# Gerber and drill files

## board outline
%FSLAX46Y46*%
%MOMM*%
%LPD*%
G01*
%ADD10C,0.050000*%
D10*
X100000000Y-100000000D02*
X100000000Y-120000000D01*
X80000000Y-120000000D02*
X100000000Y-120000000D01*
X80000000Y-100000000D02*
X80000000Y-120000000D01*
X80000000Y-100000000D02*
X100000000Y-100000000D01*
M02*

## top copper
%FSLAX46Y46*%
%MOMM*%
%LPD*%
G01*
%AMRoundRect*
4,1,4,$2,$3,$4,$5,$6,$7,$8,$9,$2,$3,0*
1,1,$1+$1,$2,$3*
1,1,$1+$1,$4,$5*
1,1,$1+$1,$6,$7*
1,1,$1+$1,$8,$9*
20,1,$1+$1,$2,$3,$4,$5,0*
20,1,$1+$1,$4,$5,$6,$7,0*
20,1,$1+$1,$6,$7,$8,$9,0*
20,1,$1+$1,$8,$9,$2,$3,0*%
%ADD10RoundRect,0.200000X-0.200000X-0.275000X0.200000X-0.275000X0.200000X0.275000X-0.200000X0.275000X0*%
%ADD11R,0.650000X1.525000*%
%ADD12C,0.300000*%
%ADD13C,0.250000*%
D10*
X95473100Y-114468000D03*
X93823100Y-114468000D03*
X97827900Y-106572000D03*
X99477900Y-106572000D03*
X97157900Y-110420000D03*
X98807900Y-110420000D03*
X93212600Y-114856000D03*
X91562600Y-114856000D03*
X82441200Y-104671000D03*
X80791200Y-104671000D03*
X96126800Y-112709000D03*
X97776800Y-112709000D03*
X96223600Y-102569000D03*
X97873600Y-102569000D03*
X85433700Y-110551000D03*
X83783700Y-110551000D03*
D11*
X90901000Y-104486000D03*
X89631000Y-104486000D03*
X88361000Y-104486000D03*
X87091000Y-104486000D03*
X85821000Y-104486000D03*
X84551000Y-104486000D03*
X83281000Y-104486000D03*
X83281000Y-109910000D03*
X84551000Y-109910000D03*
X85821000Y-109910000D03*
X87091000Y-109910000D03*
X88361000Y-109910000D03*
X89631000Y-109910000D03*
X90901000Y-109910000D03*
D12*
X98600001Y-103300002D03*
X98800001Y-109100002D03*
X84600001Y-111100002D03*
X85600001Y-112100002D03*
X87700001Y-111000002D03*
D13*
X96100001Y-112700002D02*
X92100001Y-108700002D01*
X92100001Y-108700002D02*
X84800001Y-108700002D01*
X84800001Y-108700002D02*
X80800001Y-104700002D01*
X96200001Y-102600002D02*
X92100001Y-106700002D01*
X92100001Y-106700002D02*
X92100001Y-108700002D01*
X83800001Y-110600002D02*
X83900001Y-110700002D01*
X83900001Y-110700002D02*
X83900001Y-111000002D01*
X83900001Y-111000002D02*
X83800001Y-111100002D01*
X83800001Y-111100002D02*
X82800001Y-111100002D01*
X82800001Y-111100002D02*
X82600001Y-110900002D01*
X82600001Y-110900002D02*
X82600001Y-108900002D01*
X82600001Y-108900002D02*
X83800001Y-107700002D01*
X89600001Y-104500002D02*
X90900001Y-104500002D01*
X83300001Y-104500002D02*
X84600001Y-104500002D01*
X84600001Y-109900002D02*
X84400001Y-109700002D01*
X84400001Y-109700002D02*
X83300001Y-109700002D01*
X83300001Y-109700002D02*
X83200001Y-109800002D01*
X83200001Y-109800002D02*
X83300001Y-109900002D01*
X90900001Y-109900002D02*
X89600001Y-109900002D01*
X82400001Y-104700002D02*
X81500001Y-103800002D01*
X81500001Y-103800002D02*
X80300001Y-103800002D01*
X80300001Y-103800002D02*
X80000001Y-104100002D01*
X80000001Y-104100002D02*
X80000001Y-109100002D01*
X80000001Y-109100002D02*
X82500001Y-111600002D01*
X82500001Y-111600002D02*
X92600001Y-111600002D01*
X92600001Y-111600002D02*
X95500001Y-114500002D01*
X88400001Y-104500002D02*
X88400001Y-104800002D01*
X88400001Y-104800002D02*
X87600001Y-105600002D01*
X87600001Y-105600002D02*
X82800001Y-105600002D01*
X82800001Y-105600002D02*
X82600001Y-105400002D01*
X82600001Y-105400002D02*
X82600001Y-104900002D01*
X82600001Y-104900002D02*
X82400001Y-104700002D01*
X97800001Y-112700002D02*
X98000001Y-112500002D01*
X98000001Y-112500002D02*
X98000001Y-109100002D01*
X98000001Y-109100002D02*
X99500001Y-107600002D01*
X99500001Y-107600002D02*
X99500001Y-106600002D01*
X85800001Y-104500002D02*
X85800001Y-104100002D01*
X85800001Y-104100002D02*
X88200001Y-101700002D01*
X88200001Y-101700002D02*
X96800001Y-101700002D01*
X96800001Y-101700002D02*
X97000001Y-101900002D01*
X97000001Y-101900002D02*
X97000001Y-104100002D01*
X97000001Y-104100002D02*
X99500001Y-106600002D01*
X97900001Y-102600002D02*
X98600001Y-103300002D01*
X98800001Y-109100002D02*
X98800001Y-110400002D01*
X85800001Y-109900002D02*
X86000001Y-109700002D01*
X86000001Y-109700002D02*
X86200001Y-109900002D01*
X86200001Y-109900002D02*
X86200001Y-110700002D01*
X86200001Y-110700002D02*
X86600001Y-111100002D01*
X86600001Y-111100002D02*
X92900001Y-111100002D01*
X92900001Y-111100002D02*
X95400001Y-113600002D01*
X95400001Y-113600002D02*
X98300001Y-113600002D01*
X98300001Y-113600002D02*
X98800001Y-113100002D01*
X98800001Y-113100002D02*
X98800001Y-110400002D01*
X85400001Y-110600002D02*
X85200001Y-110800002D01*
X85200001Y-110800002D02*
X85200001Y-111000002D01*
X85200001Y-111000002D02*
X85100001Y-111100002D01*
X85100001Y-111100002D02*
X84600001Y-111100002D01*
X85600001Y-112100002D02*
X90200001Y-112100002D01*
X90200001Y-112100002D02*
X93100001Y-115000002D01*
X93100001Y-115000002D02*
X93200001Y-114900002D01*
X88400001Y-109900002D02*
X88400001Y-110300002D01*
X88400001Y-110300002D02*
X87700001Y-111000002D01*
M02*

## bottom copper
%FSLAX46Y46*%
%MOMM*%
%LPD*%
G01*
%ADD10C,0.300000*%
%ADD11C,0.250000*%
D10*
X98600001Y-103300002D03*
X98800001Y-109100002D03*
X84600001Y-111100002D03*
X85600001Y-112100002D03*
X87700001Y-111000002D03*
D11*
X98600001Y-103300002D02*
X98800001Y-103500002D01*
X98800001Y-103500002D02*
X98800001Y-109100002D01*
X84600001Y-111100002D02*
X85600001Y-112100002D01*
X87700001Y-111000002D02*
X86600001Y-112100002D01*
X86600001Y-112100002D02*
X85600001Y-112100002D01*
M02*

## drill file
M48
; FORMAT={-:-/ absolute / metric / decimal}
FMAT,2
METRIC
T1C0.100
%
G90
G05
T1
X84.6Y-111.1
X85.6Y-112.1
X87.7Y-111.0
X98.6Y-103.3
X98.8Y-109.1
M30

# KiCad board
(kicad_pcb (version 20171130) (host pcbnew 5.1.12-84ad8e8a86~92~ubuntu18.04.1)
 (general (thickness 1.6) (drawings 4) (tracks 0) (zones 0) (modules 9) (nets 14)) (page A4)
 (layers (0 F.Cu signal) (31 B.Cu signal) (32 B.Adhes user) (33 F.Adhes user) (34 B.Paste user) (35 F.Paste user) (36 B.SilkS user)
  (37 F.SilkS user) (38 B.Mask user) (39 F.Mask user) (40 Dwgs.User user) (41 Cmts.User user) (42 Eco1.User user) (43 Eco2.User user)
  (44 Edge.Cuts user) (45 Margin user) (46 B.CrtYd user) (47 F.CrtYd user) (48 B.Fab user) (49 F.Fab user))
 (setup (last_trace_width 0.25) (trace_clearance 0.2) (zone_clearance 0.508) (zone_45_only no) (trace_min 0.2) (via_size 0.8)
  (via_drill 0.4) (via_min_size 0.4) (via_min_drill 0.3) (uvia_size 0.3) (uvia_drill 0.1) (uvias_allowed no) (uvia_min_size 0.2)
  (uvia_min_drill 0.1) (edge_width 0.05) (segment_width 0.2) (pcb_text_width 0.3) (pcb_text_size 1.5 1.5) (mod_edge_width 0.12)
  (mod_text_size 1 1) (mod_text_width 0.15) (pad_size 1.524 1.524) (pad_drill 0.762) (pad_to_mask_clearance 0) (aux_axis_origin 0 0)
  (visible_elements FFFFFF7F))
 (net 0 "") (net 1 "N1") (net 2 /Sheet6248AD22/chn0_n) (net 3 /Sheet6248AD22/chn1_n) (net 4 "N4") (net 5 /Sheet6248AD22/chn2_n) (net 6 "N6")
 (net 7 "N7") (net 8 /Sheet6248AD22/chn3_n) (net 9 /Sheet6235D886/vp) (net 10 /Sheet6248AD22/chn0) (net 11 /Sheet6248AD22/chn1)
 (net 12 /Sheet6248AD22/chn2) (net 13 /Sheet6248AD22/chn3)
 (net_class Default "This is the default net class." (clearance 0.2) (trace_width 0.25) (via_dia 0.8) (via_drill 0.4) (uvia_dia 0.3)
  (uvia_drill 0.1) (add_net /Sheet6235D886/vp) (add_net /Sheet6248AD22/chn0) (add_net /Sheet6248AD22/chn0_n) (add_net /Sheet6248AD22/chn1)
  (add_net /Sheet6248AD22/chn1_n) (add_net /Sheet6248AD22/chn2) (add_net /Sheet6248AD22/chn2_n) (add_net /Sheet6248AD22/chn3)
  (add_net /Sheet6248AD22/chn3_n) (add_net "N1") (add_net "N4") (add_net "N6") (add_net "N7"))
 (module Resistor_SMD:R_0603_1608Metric (layer F.Cu) (at 94.648100 114.468000)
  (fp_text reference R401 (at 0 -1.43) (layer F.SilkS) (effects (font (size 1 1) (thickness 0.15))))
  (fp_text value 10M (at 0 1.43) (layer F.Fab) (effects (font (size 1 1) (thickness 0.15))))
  (pad 2 smd roundrect (at 0.825 0) (size 0.8 0.95) (layers F.Cu F.Mask F.Paste) (roundrect_rratio 0.25) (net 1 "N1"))
  (pad 1 smd roundrect (at -0.825 0) (size 0.8 0.95) (layers F.Cu F.Mask F.Paste) (roundrect_rratio 0.25) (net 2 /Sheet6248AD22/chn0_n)))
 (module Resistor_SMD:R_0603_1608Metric (layer F.Cu) (at 98.652900 106.572000)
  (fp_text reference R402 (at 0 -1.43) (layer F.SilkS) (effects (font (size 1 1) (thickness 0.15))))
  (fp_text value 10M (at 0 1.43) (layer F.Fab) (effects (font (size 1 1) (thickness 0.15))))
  (pad 1 smd roundrect (at -0.825 0) (size 0.8 0.95) (layers F.Cu F.Mask F.Paste) (roundrect_rratio 0.25) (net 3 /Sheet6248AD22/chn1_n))
  (pad 2 smd roundrect (at 0.825 0) (size 0.8 0.95) (layers F.Cu F.Mask F.Paste) (roundrect_rratio 0.25) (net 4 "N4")))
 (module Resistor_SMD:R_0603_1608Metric (layer F.Cu) (at 97.982900 110.420000)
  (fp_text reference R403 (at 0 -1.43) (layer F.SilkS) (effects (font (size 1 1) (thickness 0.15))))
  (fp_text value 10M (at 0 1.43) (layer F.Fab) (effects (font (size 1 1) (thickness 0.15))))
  (pad 1 smd roundrect (at -0.825 0) (size 0.8 0.95) (layers F.Cu F.Mask F.Paste) (roundrect_rratio 0.25) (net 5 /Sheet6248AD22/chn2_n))
  (pad 2 smd roundrect (at 0.825 0) (size 0.8 0.95) (layers F.Cu F.Mask F.Paste) (roundrect_rratio 0.25) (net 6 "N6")))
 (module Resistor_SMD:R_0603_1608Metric (layer F.Cu) (at 92.387600 114.856000)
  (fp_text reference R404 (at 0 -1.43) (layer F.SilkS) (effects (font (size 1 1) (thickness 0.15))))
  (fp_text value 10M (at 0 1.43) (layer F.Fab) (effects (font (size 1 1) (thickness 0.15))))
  (pad 2 smd roundrect (at 0.825 0) (size 0.8 0.95) (layers F.Cu F.Mask F.Paste) (roundrect_rratio 0.25) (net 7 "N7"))
  (pad 1 smd roundrect (at -0.825 0) (size 0.8 0.95) (layers F.Cu F.Mask F.Paste) (roundrect_rratio 0.25) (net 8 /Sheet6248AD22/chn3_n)))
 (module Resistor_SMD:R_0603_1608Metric (layer F.Cu) (at 81.616200 104.671000)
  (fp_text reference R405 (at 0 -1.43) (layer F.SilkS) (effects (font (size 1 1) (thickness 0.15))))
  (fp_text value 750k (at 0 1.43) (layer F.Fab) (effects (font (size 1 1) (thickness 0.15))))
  (pad 2 smd roundrect (at 0.825 0) (size 0.8 0.95) (layers F.Cu F.Mask F.Paste) (roundrect_rratio 0.25) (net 1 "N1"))
  (pad 1 smd roundrect (at -0.825 0) (size 0.8 0.95) (layers F.Cu F.Mask F.Paste) (roundrect_rratio 0.25) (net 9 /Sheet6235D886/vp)))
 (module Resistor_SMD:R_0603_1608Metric (layer F.Cu) (at 96.951800 112.709000)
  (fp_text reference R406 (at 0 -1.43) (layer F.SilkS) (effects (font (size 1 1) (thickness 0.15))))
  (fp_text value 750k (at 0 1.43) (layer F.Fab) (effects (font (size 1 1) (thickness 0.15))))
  (pad 1 smd roundrect (at -0.825 0) (size 0.8 0.95) (layers F.Cu F.Mask F.Paste) (roundrect_rratio 0.25) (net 9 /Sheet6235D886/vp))
  (pad 2 smd roundrect (at 0.825 0) (size 0.8 0.95) (layers F.Cu F.Mask F.Paste) (roundrect_rratio 0.25) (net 4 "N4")))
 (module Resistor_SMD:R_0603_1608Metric (layer F.Cu) (at 97.048600 102.569000)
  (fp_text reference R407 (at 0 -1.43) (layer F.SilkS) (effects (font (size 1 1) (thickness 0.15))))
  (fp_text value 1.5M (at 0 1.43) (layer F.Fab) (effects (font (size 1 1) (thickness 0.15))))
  (pad 1 smd roundrect (at -0.825 0) (size 0.8 0.95) (layers F.Cu F.Mask F.Paste) (roundrect_rratio 0.25) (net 9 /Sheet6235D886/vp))
  (pad 2 smd roundrect (at 0.825 0) (size 0.8 0.95) (layers F.Cu F.Mask F.Paste) (roundrect_rratio 0.25) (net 6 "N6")))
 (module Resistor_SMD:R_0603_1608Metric (layer F.Cu) (at 84.608700 110.551000)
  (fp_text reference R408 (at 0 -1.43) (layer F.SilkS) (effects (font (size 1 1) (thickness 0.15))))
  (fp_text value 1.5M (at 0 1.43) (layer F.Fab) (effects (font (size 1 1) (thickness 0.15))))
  (pad 2 smd roundrect (at 0.825 0) (size 0.8 0.95) (layers F.Cu F.Mask F.Paste) (roundrect_rratio 0.25) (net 7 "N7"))
  (pad 1 smd roundrect (at -0.825 0) (size 0.8 0.95) (layers F.Cu F.Mask F.Paste) (roundrect_rratio 0.25) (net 9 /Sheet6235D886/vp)))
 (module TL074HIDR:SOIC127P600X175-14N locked (layer F.Cu) (at 87.091000 107.198000 270.000000)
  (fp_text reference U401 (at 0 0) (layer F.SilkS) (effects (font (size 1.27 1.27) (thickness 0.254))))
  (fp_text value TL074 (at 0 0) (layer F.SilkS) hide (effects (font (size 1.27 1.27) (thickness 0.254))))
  (pad 1 smd rect (at -2.712 -3.81) (size 0.65 1.525) (layers F.Cu F.Mask F.Paste) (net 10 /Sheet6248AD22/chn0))
  (pad 2 smd rect (at -2.712 -2.54) (size 0.65 1.525) (layers F.Cu F.Mask F.Paste) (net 10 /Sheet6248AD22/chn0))
  (pad 3 smd rect (at -2.712 -1.27) (size 0.65 1.525) (layers F.Cu F.Mask F.Paste) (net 1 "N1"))
  (pad 4 smd rect (at -2.712 0) (size 0.65 1.525) (layers F.Cu F.Mask F.Paste))
  (pad 5 smd rect (at -2.712 1.27) (size 0.65 1.525) (layers F.Cu F.Mask F.Paste) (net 4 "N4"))
  (pad 6 smd rect (at -2.712 2.54) (size 0.65 1.525) (layers F.Cu F.Mask F.Paste) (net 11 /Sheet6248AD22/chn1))
  (pad 7 smd rect (at -2.712 3.81) (size 0.65 1.525) (layers F.Cu F.Mask F.Paste) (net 11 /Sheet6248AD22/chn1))
  (pad 8 smd rect (at 2.712 3.81) (size 0.65 1.525) (layers F.Cu F.Mask F.Paste) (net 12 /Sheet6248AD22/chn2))
  (pad 9 smd rect (at 2.712 2.54) (size 0.65 1.525) (layers F.Cu F.Mask F.Paste) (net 12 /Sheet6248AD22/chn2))
  (pad 10 smd rect (at 2.712 1.27) (size 0.65 1.525) (layers F.Cu F.Mask F.Paste) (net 6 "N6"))
  (pad 11 smd rect (at 2.712 0) (size 0.65 1.525) (layers F.Cu F.Mask F.Paste))
  (pad 12 smd rect (at 2.712 -1.27) (size 0.65 1.525) (layers F.Cu F.Mask F.Paste) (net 7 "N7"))
  (pad 13 smd rect (at 2.712 -2.54) (size 0.65 1.525) (layers F.Cu F.Mask F.Paste) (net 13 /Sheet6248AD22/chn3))
  (pad 14 smd rect (at 2.712 -3.81) (size 0.65 1.525) (layers F.Cu F.Mask F.Paste) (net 13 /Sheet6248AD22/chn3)))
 (gr_line (start 100 100) (end 100 120) (layer Edge.Cuts) (width 0.05))
 (gr_line (start 80 120) (end 100 120) (layer Edge.Cuts) (width 0.05))
 (gr_line (start 80 100) (end 80 120) (layer Edge.Cuts) (width 0.05))
 (gr_line (start 80 100) (end 100 100) (layer Edge.Cuts) (width 0.05))
 (segment (start 96.100001 112.700002) (end 92.100001 108.700002) (width 0.250000) (layer F.Cu) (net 9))
 (segment (start 92.100001 108.700002) (end 84.800001 108.700002) (width 0.250000) (layer F.Cu) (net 9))
 (segment (start 84.800001 108.700002) (end 80.800001 104.700002) (width 0.250000) (layer F.Cu) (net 9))
 (segment (start 96.200001 102.600002) (end 92.100001 106.700002) (width 0.250000) (layer F.Cu) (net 9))
 (segment (start 92.100001 106.700002) (end 92.100001 108.700002) (width 0.250000) (layer F.Cu) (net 9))
 (segment (start 83.800001 110.600002) (end 83.900001 110.700002) (width 0.250000) (layer F.Cu) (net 9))
 (segment (start 83.900001 110.700002) (end 83.900001 111.000002) (width 0.250000) (layer F.Cu) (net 9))
 (segment (start 83.900001 111.000002) (end 83.800001 111.100002) (width 0.250000) (layer F.Cu) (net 9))
 (segment (start 83.800001 111.100002) (end 82.800001 111.100002) (width 0.250000) (layer F.Cu) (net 9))
 (segment (start 82.800001 111.100002) (end 82.600001 110.900002) (width 0.250000) (layer F.Cu) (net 9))
 (segment (start 82.600001 110.900002) (end 82.600001 108.900002) (width 0.250000) (layer F.Cu) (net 9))
 (segment (start 82.600001 108.900002) (end 83.800001 107.700002) (width 0.250000) (layer F.Cu) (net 9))
 (segment (start 89.600001 104.500002) (end 90.900001 104.500002) (width 0.250000) (layer F.Cu) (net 10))
 (segment (start 83.300001 104.500002) (end 84.600001 104.500002) (width 0.250000) (layer F.Cu) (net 11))
 (segment (start 84.600001 109.900002) (end 84.400001 109.700002) (width 0.250000) (layer F.Cu) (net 12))
 (segment (start 84.400001 109.700002) (end 83.300001 109.700002) (width 0.250000) (layer F.Cu) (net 12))
 (segment (start 83.300001 109.700002) (end 83.200001 109.800002) (width 0.250000) (layer F.Cu) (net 12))
 (segment (start 83.200001 109.800002) (end 83.300001 109.900002) (width 0.250000) (layer F.Cu) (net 12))
 (segment (start 90.900001 109.900002) (end 89.600001 109.900002) (width 0.250000) (layer F.Cu) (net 13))
 (segment (start 82.400001 104.700002) (end 81.500001 103.800002) (width 0.250000) (layer F.Cu) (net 1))
 (segment (start 81.500001 103.800002) (end 80.300001 103.800002) (width 0.250000) (layer F.Cu) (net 1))
 (segment (start 80.300001 103.800002) (end 80.000001 104.100002) (width 0.250000) (layer F.Cu) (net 1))
 (segment (start 80.000001 104.100002) (end 80.000001 109.100002) (width 0.250000) (layer F.Cu) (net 1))
 (segment (start 80.000001 109.100002) (end 82.500001 111.600002) (width 0.250000) (layer F.Cu) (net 1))
 (segment (start 82.500001 111.600002) (end 92.600001 111.600002) (width 0.250000) (layer F.Cu) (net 1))
 (segment (start 92.600001 111.600002) (end 95.500001 114.500002) (width 0.250000) (layer F.Cu) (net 1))
 (segment (start 88.400001 104.500002) (end 88.400001 104.800002) (width 0.250000) (layer F.Cu) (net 1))
 (segment (start 88.400001 104.800002) (end 87.600001 105.600002) (width 0.250000) (layer F.Cu) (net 1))
 (segment (start 87.600001 105.600002) (end 82.800001 105.600002) (width 0.250000) (layer F.Cu) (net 1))
 (segment (start 82.800001 105.600002) (end 82.600001 105.400002) (width 0.250000) (layer F.Cu) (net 1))
 (segment (start 82.600001 105.400002) (end 82.600001 104.900002) (width 0.250000) (layer F.Cu) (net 1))
 (segment (start 82.600001 104.900002) (end 82.400001 104.700002) (width 0.250000) (layer F.Cu) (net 1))
 (segment (start 97.800001 112.700002) (end 98.000001 112.500002) (width 0.250000) (layer F.Cu) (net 4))
 (segment (start 98.000001 112.500002) (end 98.000001 109.100002) (width 0.250000) (layer F.Cu) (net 4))
 (segment (start 98.000001 109.100002) (end 99.500001 107.600002) (width 0.250000) (layer F.Cu) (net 4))
 (segment (start 99.500001 107.600002) (end 99.500001 106.600002) (width 0.250000) (layer F.Cu) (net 4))
 (segment (start 85.800001 104.500002) (end 85.800001 104.100002) (width 0.250000) (layer F.Cu) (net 4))
 (segment (start 85.800001 104.100002) (end 88.200001 101.700002) (width 0.250000) (layer F.Cu) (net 4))
 (segment (start 88.200001 101.700002) (end 96.800001 101.700002) (width 0.250000) (layer F.Cu) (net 4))
 (segment (start 96.800001 101.700002) (end 97.000001 101.900002) (width 0.250000) (layer F.Cu) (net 4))
 (segment (start 97.000001 101.900002) (end 97.000001 104.100002) (width 0.250000) (layer F.Cu) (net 4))
 (segment (start 97.000001 104.100002) (end 99.500001 106.600002) (width 0.250000) (layer F.Cu) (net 4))
 (segment (start 97.900001 102.600002) (end 98.600001 103.300002) (width 0.250000) (layer F.Cu) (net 6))
 (segment (start 98.600001 103.300002) (end 98.800001 103.500002) (width 0.250000) (layer B.Cu) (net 6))
 (segment (start 98.800001 103.500002) (end 98.800001 109.100002) (width 0.250000) (layer B.Cu) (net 6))
 (segment (start 98.800001 109.100002) (end 98.800001 110.400002) (width 0.250000) (layer F.Cu) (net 6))
 (segment (start 85.800001 109.900002) (end 86.000001 109.700002) (width 0.250000) (layer F.Cu) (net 6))
 (segment (start 86.000001 109.700002) (end 86.200001 109.900002) (width 0.250000) (layer F.Cu) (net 6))
 (segment (start 86.200001 109.900002) (end 86.200001 110.700002) (width 0.250000) (layer F.Cu) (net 6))
 (segment (start 86.200001 110.700002) (end 86.600001 111.100002) (width 0.250000) (layer F.Cu) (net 6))
 (segment (start 86.600001 111.100002) (end 92.900001 111.100002) (width 0.250000) (layer F.Cu) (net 6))
 (segment (start 92.900001 111.100002) (end 95.400001 113.600002) (width 0.250000) (layer F.Cu) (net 6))
 (segment (start 95.400001 113.600002) (end 98.300001 113.600002) (width 0.250000) (layer F.Cu) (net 6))
 (segment (start 98.300001 113.600002) (end 98.800001 113.100002) (width 0.250000) (layer F.Cu) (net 6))
 (segment (start 98.800001 113.100002) (end 98.800001 110.400002) (width 0.250000) (layer F.Cu) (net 6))
 (via micro (at 98.600001 103.300002) (size 0.300000) (drill 0.100000) (layers F.Cu B.Cu) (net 6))
 (via micro (at 98.800001 109.100002) (size 0.300000) (drill 0.100000) (layers F.Cu B.Cu) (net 6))
 (segment (start 85.400001 110.600002) (end 85.200001 110.800002) (width 0.250000) (layer F.Cu) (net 7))
 (segment (start 85.200001 110.800002) (end 85.200001 111.000002) (width 0.250000) (layer F.Cu) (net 7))
 (segment (start 85.200001 111.000002) (end 85.100001 111.100002) (width 0.250000) (layer F.Cu) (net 7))
 (segment (start 85.100001 111.100002) (end 84.600001 111.100002) (width 0.250000) (layer F.Cu) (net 7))
 (segment (start 84.600001 111.100002) (end 85.600001 112.100002) (width 0.250000) (layer B.Cu) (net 7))
 (segment (start 85.600001 112.100002) (end 90.200001 112.100002) (width 0.250000) (layer F.Cu) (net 7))
 (segment (start 90.200001 112.100002) (end 93.100001 115.000002) (width 0.250000) (layer F.Cu) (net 7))
 (segment (start 93.100001 115.000002) (end 93.200001 114.900002) (width 0.250000) (layer F.Cu) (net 7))
 (segment (start 88.400001 109.900002) (end 88.400001 110.300002) (width 0.250000) (layer F.Cu) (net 7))
 (segment (start 88.400001 110.300002) (end 87.700001 111.000002) (width 0.250000) (layer F.Cu) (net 7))
 (segment (start 87.700001 111.000002) (end 86.600001 112.100002) (width 0.250000) (layer B.Cu) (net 7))
 (segment (start 86.600001 112.100002) (end 85.600001 112.100002) (width 0.250000) (layer B.Cu) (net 7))
 (via micro (at 84.600001 111.100002) (size 0.300000) (drill 0.100000) (layers F.Cu B.Cu) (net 7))
 (via micro (at 85.600001 112.100002) (size 0.300000) (drill 0.100000) (layers F.Cu B.Cu) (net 7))
 (via micro (at 87.700001 111.000002) (size 0.300000) (drill 0.100000) (layers F.Cu B.Cu) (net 7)))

